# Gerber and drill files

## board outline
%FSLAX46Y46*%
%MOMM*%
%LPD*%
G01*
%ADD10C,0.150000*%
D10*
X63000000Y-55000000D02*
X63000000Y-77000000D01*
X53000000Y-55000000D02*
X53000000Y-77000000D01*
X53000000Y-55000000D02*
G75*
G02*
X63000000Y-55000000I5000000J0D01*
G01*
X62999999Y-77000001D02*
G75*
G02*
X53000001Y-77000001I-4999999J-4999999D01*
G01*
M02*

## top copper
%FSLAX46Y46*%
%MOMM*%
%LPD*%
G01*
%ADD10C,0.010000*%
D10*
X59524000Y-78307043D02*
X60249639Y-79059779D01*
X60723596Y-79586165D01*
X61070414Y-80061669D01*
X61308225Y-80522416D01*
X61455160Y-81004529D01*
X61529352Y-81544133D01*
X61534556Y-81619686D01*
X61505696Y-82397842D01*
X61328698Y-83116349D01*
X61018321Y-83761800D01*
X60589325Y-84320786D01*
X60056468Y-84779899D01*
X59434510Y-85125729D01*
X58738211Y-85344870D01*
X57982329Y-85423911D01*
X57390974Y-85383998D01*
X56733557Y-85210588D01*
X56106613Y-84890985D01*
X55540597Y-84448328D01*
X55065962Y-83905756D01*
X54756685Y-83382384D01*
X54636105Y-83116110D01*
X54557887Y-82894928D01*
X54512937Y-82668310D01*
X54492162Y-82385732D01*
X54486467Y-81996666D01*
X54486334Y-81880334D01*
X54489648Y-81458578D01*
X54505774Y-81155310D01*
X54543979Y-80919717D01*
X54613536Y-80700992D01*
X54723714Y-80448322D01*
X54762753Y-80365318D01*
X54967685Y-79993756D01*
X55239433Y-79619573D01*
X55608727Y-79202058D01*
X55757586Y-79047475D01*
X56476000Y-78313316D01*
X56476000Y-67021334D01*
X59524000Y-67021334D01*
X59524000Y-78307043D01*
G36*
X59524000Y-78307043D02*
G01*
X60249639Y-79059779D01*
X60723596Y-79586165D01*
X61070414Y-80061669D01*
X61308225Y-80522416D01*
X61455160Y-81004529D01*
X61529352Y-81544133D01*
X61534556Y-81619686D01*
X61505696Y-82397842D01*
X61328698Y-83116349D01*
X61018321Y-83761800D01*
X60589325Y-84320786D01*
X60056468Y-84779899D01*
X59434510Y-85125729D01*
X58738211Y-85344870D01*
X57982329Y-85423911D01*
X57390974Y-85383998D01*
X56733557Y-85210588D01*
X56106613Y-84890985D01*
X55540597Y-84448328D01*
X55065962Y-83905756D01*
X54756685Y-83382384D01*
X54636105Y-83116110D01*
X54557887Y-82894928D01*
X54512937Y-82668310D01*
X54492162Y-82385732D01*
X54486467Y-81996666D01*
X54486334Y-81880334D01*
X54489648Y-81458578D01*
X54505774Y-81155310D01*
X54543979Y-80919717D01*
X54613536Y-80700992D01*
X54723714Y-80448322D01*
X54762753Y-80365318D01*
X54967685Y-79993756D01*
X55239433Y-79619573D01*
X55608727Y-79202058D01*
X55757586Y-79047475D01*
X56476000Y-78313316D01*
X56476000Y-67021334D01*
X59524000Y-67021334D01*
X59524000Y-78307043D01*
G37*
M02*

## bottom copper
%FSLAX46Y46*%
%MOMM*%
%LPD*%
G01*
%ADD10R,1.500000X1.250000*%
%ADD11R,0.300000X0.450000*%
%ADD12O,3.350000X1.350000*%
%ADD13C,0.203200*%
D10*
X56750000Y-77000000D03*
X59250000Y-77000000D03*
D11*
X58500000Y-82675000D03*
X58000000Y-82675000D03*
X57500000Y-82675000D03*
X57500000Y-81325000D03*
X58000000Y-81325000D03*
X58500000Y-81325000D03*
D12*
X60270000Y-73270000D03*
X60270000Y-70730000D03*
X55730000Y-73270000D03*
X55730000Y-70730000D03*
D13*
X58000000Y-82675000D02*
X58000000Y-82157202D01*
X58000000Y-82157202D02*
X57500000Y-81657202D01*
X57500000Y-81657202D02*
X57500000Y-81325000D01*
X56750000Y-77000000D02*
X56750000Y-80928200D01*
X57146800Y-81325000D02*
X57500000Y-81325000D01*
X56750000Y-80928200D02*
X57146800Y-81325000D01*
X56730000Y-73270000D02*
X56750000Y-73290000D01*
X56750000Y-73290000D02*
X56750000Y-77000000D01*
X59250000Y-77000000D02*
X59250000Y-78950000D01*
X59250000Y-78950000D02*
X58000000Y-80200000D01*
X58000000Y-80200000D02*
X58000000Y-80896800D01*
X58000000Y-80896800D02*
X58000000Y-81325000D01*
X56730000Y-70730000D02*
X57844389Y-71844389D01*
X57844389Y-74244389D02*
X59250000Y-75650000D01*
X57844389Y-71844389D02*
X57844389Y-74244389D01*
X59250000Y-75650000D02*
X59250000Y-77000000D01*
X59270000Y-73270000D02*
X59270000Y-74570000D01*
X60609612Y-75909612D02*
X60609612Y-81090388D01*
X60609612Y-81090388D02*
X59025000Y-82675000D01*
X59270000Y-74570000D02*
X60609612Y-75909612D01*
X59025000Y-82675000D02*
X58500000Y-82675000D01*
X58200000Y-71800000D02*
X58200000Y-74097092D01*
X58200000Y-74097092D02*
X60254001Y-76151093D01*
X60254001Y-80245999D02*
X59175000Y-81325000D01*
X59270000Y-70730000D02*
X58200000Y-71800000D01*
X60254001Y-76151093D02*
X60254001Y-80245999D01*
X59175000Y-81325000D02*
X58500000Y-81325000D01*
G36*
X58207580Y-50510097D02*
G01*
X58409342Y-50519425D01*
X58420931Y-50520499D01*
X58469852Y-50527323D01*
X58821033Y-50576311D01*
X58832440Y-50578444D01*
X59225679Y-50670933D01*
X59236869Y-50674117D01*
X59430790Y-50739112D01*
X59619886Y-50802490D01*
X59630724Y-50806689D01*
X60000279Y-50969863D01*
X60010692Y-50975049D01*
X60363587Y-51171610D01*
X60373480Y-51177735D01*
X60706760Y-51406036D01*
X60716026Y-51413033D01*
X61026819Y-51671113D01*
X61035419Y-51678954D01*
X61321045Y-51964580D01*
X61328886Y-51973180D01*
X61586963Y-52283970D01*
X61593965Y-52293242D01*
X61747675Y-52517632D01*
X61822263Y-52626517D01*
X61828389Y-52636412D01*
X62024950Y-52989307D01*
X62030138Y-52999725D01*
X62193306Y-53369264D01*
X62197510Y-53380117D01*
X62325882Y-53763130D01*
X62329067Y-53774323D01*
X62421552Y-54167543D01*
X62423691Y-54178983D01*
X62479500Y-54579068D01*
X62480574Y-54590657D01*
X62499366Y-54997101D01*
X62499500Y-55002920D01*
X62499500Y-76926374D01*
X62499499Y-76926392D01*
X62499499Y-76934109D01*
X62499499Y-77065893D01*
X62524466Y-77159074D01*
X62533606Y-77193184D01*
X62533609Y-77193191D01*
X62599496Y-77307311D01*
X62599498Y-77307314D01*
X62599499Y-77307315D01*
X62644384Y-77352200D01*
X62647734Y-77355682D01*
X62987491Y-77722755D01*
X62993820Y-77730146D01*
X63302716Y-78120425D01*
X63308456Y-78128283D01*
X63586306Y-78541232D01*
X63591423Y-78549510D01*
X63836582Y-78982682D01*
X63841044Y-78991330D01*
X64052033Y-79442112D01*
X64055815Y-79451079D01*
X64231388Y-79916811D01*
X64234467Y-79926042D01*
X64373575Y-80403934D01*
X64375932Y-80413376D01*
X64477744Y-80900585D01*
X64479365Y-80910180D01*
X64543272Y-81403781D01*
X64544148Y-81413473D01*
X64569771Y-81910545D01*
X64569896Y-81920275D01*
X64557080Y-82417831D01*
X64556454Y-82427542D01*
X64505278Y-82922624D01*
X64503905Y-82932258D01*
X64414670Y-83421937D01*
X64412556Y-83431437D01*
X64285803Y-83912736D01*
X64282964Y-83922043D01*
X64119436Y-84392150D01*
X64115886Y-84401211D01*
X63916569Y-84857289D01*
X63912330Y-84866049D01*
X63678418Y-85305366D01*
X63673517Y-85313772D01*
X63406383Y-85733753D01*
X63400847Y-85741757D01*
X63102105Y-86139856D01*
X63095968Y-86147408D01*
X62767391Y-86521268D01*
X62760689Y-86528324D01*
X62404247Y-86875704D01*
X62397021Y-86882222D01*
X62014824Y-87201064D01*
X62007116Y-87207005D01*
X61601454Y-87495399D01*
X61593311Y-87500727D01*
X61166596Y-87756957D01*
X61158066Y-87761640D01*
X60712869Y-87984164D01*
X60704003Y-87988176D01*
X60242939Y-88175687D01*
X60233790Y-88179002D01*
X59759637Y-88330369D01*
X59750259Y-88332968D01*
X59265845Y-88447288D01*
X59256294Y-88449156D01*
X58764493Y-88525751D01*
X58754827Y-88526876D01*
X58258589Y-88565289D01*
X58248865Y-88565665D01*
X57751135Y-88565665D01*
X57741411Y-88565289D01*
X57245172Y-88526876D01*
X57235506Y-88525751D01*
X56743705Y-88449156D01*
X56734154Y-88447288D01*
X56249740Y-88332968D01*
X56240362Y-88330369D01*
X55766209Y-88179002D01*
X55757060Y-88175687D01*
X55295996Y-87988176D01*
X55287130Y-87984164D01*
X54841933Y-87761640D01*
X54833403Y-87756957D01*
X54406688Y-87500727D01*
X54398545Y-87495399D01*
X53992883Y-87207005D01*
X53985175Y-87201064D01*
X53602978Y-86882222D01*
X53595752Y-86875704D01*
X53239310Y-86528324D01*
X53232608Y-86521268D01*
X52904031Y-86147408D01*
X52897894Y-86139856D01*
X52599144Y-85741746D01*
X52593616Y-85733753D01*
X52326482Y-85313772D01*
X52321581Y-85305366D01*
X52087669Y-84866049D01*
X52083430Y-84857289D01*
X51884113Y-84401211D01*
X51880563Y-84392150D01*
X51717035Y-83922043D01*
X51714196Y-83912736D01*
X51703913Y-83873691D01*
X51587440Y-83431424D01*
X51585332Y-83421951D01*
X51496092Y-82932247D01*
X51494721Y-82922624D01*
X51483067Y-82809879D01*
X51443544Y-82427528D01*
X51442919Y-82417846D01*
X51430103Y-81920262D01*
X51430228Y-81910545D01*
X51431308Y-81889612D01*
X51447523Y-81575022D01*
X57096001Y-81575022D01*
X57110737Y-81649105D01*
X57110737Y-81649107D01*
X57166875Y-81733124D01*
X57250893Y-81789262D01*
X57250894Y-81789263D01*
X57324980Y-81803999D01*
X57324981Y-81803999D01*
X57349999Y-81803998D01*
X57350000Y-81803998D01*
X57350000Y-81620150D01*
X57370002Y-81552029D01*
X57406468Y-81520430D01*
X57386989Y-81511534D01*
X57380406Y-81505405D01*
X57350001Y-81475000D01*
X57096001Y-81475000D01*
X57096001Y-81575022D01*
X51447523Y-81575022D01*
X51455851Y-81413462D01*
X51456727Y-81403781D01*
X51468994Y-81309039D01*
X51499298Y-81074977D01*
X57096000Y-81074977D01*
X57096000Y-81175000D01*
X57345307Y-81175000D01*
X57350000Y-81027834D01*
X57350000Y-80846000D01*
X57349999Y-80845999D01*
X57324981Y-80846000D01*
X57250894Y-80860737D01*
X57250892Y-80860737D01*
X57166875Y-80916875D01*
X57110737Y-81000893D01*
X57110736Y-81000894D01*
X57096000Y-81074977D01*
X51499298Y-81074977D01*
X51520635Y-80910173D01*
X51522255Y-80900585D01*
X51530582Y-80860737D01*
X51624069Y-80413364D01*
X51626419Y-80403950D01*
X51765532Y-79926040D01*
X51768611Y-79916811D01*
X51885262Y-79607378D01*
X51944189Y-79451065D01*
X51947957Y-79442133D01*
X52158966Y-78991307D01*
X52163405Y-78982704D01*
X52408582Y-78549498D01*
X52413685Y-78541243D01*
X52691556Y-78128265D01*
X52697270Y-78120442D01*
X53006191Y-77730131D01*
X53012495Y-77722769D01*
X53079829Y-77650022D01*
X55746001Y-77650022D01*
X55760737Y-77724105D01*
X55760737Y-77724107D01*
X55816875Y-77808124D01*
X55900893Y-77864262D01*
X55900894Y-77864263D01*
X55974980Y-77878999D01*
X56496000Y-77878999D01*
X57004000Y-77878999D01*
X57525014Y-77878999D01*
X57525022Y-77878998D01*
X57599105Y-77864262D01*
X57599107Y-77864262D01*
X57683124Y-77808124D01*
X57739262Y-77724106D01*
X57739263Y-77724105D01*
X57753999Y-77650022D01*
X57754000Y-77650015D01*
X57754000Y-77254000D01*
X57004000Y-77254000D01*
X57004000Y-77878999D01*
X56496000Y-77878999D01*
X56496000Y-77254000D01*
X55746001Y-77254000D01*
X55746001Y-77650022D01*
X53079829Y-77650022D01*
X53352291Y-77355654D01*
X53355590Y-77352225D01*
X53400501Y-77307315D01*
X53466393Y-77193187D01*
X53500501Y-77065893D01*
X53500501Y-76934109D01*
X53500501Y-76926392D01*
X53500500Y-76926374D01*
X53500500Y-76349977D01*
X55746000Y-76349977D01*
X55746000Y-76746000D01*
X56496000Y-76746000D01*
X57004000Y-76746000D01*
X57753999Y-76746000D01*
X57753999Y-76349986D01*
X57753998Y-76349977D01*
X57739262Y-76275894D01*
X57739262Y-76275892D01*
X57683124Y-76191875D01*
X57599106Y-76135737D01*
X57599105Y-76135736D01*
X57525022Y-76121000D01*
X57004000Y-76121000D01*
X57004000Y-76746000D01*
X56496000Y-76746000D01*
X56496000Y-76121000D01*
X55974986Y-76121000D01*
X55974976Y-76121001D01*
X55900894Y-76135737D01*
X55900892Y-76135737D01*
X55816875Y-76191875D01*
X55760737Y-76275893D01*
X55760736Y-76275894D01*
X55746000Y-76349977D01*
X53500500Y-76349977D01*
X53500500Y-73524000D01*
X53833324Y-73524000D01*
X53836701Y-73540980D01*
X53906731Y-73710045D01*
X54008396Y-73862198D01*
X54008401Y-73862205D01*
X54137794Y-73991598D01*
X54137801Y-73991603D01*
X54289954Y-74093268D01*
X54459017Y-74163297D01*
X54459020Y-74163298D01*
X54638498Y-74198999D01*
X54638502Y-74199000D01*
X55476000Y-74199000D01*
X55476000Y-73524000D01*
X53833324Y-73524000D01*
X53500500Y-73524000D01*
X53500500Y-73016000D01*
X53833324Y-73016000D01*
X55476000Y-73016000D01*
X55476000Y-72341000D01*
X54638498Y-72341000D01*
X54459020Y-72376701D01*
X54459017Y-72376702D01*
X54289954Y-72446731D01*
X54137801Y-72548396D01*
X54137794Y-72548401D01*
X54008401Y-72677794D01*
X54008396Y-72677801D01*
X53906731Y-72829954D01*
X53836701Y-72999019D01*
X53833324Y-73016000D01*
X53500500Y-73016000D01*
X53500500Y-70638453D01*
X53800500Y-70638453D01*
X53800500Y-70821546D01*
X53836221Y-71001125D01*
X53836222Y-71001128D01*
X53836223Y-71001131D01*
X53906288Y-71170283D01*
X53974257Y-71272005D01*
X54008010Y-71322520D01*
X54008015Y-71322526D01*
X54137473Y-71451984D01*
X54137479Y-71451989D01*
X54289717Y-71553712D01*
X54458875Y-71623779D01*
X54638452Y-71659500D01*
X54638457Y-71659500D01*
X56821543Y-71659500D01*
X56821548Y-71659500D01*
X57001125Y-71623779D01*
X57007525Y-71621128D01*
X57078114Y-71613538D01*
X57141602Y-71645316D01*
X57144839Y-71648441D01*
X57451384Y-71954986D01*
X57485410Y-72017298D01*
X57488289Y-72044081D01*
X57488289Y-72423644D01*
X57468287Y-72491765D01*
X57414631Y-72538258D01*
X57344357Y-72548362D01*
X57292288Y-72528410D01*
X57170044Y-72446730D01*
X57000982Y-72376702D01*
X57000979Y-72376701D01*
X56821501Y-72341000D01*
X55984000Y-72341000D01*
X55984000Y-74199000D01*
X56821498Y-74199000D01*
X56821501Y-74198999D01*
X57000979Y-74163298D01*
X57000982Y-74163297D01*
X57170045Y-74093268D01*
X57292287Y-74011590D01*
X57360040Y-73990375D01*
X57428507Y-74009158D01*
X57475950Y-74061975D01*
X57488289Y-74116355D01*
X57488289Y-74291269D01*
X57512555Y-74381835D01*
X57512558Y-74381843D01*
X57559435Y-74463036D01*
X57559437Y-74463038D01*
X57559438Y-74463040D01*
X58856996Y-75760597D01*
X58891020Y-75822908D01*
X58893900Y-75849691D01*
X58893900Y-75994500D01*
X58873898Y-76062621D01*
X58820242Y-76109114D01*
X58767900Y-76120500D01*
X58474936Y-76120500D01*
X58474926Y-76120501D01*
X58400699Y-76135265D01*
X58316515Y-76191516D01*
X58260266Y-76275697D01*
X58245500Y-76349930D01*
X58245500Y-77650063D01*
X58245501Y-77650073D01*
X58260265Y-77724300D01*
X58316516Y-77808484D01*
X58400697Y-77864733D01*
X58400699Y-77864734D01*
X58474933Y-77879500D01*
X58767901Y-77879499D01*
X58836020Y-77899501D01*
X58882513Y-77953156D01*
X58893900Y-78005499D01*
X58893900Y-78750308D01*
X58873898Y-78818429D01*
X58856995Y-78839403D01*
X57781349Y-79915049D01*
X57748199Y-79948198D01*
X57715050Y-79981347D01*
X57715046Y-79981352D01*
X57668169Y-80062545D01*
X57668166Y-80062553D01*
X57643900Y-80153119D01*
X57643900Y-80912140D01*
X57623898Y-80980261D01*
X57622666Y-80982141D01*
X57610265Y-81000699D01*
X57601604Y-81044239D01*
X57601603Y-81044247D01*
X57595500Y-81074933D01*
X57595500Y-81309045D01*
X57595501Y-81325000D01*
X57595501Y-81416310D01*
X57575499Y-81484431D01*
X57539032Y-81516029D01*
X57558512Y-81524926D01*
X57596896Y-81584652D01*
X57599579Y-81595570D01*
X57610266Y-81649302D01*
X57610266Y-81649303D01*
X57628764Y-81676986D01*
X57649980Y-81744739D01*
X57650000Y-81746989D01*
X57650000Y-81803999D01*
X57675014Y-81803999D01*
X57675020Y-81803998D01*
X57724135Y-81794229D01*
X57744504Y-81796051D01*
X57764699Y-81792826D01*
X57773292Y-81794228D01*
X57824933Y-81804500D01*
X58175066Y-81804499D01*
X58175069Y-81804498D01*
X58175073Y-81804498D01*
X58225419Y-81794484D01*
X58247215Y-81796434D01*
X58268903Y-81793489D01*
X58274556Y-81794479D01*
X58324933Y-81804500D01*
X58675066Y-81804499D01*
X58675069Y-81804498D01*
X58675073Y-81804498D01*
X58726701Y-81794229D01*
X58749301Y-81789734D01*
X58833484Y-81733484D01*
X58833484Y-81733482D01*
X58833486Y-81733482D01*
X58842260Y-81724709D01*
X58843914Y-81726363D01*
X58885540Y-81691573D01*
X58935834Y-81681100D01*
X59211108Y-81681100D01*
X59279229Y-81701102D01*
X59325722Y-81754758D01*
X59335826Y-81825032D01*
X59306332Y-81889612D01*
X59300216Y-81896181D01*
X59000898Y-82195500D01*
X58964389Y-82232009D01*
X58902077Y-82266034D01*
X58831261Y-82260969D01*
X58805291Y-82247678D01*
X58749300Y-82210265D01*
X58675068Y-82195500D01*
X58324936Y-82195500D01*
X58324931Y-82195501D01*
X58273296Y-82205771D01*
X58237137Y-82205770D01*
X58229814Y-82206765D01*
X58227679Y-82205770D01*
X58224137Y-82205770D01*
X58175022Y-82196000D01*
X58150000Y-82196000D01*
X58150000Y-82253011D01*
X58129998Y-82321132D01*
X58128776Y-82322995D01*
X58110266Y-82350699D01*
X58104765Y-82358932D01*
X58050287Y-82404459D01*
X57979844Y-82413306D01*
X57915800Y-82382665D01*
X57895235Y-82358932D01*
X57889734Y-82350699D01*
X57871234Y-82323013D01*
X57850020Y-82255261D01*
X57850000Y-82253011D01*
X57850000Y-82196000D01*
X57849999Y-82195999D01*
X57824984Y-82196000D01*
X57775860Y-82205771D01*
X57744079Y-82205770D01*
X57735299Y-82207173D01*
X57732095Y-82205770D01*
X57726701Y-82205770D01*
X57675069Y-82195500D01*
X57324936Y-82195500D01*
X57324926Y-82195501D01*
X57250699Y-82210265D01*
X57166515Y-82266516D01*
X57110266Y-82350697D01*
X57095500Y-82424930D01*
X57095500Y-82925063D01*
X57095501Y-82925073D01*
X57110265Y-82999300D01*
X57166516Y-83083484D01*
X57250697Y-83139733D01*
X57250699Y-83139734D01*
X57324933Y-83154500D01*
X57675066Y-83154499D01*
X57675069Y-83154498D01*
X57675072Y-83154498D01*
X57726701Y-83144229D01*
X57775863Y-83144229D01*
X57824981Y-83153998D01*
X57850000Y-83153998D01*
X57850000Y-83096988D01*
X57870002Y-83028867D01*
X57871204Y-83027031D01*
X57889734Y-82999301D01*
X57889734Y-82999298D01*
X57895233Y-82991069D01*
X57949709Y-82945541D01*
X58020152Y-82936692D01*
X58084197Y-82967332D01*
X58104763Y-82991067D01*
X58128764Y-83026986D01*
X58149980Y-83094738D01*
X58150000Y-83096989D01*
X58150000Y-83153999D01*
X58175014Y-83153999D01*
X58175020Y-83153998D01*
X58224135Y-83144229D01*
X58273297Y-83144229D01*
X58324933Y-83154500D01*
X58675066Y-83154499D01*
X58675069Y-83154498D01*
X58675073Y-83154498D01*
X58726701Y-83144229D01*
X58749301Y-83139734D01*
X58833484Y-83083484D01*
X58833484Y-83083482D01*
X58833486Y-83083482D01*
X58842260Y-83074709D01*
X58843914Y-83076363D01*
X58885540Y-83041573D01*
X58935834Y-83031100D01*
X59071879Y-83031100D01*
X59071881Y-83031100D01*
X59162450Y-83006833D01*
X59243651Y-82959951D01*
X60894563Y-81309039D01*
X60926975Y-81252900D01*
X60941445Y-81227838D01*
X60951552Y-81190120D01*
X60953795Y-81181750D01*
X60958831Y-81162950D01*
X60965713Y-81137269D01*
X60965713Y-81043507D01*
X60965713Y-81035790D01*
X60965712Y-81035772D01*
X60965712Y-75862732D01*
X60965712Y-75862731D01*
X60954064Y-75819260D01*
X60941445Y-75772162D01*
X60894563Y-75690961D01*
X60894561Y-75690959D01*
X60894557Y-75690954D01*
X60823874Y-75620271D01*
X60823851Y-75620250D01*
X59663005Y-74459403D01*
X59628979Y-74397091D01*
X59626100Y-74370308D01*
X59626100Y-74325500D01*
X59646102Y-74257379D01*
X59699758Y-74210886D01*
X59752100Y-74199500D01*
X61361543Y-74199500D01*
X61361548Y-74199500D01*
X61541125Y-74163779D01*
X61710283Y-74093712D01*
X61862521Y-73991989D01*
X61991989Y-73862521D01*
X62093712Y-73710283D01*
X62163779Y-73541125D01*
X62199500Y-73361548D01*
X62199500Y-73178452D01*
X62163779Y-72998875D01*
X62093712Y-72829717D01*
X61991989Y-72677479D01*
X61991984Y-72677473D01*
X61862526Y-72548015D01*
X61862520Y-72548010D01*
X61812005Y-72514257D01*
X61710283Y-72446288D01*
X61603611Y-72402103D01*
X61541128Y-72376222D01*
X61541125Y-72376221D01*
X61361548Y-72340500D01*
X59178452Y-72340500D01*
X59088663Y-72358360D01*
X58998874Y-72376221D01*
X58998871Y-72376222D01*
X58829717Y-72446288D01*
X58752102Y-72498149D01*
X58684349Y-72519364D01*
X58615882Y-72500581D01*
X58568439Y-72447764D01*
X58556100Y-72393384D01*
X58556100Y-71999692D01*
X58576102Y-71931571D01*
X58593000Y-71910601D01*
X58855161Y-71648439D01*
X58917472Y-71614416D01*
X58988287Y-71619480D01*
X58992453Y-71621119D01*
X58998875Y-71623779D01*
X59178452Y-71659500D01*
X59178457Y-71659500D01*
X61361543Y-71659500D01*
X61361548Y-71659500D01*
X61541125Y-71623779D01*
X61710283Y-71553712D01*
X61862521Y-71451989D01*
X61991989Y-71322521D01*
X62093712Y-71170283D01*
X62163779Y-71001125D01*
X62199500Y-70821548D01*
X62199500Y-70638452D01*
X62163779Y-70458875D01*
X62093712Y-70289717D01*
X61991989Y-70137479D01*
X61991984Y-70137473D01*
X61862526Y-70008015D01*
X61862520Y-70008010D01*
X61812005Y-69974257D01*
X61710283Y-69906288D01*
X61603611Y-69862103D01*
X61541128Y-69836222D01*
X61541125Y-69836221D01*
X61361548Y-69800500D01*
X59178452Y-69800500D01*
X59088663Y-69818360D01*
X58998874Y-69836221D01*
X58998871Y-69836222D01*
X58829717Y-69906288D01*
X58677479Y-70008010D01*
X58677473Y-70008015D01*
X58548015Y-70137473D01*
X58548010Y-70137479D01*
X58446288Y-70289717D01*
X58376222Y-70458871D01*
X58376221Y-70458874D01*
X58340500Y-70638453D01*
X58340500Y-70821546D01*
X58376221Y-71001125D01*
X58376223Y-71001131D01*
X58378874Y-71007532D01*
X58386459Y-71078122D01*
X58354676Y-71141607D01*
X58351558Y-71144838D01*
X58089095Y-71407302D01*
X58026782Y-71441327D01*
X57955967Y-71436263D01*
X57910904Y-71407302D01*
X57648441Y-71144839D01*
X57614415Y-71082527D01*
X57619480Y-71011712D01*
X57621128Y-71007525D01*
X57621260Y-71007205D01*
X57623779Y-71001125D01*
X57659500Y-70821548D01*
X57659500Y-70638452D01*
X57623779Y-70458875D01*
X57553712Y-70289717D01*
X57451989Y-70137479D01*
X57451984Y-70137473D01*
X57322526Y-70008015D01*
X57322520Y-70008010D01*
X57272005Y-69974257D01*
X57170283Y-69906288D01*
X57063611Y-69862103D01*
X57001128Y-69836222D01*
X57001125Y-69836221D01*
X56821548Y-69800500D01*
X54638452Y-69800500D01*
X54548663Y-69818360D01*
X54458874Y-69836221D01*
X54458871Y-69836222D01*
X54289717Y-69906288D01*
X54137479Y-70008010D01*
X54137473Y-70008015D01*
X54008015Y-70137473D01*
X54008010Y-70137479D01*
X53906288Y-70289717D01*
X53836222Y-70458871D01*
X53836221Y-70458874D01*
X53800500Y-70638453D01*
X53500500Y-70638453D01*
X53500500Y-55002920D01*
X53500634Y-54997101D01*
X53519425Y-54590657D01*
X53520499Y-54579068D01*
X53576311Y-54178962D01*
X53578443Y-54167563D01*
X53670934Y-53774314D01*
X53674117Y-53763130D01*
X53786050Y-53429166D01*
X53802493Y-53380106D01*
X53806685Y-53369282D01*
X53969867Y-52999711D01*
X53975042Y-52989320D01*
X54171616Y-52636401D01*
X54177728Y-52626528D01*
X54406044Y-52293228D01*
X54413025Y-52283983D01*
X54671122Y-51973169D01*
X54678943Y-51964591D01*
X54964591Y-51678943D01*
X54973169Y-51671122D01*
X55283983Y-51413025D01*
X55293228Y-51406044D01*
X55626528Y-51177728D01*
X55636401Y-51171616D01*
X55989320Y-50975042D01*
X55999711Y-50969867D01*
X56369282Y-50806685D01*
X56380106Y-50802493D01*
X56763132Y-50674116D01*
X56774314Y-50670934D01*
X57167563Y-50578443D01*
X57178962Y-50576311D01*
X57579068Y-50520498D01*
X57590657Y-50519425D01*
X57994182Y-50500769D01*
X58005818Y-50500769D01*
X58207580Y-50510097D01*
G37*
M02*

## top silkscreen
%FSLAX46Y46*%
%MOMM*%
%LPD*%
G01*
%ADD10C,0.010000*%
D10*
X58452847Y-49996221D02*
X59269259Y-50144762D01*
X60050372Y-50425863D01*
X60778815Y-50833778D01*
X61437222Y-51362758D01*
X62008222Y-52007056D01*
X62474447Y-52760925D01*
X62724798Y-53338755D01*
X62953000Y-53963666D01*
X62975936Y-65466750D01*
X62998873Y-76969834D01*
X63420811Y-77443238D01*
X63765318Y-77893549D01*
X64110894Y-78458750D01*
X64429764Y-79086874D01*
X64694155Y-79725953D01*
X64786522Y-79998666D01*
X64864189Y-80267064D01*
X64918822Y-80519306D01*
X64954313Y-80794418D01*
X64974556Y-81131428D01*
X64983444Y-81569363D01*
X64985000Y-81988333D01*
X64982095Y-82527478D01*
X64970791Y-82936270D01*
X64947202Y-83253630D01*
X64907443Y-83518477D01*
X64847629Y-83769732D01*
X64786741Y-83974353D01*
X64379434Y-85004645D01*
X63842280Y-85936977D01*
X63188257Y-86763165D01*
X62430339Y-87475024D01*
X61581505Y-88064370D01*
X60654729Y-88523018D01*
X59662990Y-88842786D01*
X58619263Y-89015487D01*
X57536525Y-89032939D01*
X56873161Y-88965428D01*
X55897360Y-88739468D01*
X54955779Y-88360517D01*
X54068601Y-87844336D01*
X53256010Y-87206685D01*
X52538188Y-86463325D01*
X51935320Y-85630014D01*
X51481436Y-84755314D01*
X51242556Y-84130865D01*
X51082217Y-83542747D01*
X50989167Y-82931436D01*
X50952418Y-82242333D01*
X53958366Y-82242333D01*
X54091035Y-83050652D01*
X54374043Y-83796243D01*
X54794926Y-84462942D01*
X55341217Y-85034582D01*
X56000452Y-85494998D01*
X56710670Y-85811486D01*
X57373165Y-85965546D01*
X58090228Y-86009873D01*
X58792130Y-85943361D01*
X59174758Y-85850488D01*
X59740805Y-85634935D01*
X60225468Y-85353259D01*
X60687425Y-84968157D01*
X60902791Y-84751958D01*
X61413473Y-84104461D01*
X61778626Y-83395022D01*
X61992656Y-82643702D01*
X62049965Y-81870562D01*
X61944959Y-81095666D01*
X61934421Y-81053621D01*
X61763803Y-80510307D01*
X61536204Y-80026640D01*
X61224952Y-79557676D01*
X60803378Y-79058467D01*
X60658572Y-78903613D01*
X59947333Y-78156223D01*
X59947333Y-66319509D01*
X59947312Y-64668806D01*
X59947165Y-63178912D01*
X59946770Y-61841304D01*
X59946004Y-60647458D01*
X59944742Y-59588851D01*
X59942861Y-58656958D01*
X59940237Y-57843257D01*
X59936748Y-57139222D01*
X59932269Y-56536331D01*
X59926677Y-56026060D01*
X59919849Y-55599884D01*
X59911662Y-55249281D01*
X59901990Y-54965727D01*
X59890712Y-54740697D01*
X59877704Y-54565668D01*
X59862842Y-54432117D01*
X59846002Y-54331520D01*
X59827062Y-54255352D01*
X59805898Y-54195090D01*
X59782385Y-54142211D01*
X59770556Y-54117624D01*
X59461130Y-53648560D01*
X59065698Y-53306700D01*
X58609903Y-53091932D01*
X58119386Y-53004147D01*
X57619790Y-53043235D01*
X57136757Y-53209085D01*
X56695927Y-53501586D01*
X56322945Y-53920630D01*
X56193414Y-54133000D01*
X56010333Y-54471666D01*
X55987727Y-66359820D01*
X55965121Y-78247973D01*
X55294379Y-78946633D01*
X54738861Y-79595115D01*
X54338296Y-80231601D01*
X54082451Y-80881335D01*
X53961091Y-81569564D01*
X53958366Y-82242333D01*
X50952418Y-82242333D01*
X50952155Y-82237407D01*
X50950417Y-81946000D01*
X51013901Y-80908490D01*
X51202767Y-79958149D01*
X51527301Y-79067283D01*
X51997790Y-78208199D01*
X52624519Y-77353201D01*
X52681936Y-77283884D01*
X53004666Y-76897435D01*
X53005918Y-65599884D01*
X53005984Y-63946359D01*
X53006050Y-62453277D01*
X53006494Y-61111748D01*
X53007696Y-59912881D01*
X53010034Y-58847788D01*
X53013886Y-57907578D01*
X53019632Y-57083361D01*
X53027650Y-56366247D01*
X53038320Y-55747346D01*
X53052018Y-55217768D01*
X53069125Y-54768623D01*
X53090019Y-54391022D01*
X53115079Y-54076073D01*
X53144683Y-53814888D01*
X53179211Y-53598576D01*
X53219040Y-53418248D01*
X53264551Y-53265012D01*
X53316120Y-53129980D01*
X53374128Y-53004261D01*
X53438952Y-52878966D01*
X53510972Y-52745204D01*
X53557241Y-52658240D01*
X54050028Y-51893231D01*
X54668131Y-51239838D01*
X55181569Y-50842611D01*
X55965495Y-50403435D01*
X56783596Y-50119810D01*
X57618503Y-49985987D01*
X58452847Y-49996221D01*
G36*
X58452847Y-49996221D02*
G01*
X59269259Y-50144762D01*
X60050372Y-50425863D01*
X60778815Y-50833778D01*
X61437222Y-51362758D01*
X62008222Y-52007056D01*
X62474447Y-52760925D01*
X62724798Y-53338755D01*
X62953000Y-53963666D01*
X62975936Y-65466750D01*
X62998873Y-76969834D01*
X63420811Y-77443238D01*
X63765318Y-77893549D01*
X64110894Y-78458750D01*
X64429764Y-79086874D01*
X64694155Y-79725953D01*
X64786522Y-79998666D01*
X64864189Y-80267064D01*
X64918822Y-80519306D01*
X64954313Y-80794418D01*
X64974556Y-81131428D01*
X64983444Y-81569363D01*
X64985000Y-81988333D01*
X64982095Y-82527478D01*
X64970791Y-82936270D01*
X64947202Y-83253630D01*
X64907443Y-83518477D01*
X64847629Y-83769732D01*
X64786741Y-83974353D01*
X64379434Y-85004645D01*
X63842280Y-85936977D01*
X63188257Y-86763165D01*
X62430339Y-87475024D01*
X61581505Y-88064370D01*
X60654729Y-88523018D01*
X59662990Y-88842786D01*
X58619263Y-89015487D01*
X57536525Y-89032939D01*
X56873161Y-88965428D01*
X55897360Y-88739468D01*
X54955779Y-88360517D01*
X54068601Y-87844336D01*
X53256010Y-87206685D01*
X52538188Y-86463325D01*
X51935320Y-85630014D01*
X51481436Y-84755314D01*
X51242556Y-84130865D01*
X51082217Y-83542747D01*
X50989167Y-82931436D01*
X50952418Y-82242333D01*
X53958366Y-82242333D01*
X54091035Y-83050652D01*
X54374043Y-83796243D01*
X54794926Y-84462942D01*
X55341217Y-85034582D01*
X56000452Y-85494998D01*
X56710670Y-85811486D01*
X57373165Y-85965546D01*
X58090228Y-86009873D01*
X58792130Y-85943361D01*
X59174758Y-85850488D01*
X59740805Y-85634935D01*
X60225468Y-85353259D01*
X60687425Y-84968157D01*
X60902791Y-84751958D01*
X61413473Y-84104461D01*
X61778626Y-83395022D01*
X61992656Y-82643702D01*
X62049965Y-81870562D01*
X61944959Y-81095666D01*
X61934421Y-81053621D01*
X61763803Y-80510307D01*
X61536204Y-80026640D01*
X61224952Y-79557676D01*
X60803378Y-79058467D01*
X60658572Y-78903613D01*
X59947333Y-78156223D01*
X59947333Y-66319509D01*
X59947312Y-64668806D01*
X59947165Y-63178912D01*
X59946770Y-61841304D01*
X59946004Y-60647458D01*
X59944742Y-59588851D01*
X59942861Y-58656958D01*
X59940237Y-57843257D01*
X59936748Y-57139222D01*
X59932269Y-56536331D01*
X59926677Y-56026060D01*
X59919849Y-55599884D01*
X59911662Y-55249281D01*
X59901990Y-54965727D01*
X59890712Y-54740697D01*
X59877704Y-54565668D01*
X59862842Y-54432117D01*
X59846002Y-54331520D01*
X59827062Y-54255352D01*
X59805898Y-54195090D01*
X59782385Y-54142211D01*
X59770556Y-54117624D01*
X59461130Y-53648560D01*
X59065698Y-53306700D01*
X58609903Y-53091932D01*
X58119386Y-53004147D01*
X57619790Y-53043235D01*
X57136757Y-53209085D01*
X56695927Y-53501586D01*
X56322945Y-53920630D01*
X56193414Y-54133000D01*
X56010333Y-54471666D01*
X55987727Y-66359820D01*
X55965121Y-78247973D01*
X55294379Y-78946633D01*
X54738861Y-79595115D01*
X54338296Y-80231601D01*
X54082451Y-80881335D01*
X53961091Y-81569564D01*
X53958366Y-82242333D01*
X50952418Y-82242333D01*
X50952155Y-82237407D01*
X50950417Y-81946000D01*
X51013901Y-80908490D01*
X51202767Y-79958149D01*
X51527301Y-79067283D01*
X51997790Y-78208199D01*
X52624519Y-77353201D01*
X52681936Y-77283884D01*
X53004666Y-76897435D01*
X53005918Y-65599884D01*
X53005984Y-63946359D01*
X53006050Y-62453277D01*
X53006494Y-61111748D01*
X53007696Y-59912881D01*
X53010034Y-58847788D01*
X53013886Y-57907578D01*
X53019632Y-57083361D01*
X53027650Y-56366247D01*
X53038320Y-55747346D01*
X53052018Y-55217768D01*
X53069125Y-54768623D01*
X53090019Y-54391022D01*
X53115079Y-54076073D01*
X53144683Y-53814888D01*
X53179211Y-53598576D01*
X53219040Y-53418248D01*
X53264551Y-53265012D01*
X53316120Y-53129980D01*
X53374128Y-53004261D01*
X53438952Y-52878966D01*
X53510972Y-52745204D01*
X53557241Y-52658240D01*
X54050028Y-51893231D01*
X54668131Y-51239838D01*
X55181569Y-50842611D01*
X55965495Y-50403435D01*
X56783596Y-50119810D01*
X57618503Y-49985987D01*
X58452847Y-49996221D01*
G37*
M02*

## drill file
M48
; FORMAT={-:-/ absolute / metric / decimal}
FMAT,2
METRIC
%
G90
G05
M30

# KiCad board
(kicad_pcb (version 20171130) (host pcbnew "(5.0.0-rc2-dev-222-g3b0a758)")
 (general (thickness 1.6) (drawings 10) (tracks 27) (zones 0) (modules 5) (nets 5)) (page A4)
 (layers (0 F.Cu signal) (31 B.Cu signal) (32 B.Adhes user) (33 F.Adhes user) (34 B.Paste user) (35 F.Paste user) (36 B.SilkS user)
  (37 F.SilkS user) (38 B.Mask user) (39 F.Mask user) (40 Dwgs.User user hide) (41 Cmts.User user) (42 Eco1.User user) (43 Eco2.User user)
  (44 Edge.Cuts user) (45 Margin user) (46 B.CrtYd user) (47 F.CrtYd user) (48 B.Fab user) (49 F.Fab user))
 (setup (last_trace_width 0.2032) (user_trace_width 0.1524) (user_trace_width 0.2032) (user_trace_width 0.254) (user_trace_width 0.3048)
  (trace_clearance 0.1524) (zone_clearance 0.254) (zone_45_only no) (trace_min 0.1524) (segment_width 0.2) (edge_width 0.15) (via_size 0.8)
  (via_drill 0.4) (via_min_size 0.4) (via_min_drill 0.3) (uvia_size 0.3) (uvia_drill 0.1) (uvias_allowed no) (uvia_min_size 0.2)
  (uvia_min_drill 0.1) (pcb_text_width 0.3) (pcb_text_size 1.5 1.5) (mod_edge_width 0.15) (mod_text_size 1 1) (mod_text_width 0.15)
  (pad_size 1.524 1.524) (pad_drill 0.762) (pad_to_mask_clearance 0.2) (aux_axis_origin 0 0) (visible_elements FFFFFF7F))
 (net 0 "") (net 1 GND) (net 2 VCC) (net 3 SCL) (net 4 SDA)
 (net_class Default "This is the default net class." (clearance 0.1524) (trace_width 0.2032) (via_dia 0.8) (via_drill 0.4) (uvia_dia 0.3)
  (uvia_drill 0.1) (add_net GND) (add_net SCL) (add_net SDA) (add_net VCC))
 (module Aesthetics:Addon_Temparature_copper (layer F.Cu) (at 58 76.25)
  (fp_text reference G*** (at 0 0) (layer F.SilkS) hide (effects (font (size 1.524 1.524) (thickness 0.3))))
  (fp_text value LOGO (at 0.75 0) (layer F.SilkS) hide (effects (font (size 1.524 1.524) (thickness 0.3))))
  (fp_poly
   (pts (xy 1.524 2.057043) (xy 2.249639 2.809779) (xy 2.723596 3.336165) (xy 3.070414 3.811669) (xy 3.308225 4.272416)
    (xy 3.45516 4.754529) (xy 3.529352 5.294133) (xy 3.534556 5.369686) (xy 3.505696 6.147842) (xy 3.328698 6.866349) (xy 3.018321 7.5118)
    (xy 2.589325 8.070786) (xy 2.056468 8.529899) (xy 1.43451 8.875729) (xy 0.738211 9.09487) (xy -0.017671 9.173911)
    (xy -0.609026 9.133998) (xy -1.266443 8.960588) (xy -1.893387 8.640985) (xy -2.459403 8.198328) (xy -2.934038 7.655756)
    (xy -3.243315 7.132384) (xy -3.363895 6.86611) (xy -3.442113 6.644928) (xy -3.487063 6.41831) (xy -3.507838 6.135732)
    (xy -3.513533 5.746666) (xy -3.513666 5.630334) (xy -3.510352 5.208578) (xy -3.494226 4.90531) (xy -3.456021 4.669717)
    (xy -3.386464 4.450992) (xy -3.276286 4.198322) (xy -3.237247 4.115318) (xy -3.032315 3.743756) (xy -2.760567 3.369573)
    (xy -2.391273 2.952058) (xy -2.242414 2.797475) (xy -1.524 2.063316) (xy -1.524 -9.228666) (xy 1.524 -9.228666) (xy 1.524 2.057043))
   (layer F.Cu) (width 0.01)))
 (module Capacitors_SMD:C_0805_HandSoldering (layer B.Cu) (at 58 77 180)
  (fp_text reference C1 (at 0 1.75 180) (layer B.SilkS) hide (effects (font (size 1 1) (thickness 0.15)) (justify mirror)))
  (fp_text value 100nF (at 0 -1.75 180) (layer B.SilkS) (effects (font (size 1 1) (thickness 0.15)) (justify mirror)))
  (pad 2 smd rect (at 1.25 0 180) (size 1.5 1.25) (layers B.Cu B.Paste B.Mask) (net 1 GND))
  (pad 1 smd rect (at -1.25 0 180) (size 1.5 1.25) (layers B.Cu B.Paste B.Mask) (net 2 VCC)))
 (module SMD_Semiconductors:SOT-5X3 (layer B.Cu) (at 58 82 90)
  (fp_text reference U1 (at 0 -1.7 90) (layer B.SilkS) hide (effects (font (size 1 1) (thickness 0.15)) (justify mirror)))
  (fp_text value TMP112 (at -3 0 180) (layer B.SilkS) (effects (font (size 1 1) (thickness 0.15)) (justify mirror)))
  (pad 1 smd rect (at -0.675 0.5 90) (size 0.45 0.3) (layers B.Cu B.Paste B.Mask) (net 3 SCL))
  (pad 2 smd rect (at -0.675 0 90) (size 0.45 0.3) (layers B.Cu B.Paste B.Mask) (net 1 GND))
  (pad 3 smd rect (at -0.675 -0.5 90) (size 0.45 0.3) (layers B.Cu B.Paste B.Mask))
  (pad 4 smd rect (at 0.675 -0.5 90) (size 0.45 0.3) (layers B.Cu B.Paste B.Mask) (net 1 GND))
  (pad 5 smd rect (at 0.675 0 90) (size 0.45 0.3) (layers B.Cu B.Paste B.Mask) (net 2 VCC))
  (pad 6 smd rect (at 0.675 0.5 90) (size 0.45 0.3) (layers B.Cu B.Paste B.Mask) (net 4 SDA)))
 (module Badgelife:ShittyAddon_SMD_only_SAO (layer F.Cu) (at 56.73 70.73)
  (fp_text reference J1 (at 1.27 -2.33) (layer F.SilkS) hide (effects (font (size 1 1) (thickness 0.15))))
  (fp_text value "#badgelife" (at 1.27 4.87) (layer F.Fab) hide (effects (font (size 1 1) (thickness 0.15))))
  (pad 3 smd oval (at 2.54 2.54) (size 3.35 1.35) (drill (offset 1 0)) (layers B.Cu B.Paste B.Mask) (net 3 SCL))
  (pad 4 smd oval (at 2.54 0) (size 3.35 1.35) (drill (offset 1 0)) (layers B.Cu B.Paste B.Mask) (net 4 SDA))
  (pad 2 smd oval (at 0 2.54) (size 3.35 1.35) (drill (offset -1 0)) (layers B.Cu B.Paste B.Mask) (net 1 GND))
  (pad 1 smd oval (at 0 0) (size 3.35 1.35) (drill (offset -1 0)) (layers B.Cu B.Paste B.Mask) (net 2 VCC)))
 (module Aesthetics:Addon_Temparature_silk (layer F.Cu) (at 58 69.5)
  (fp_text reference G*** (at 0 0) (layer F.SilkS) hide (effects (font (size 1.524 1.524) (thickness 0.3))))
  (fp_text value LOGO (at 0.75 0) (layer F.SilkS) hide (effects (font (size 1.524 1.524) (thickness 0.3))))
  (fp_poly
   (pts (xy 0.452847 -19.503779) (xy 1.269259 -19.355238) (xy 2.050372 -19.074137) (xy 2.778815 -18.666222) (xy 3.437222 -18.137242)
    (xy 4.008222 -17.492944) (xy 4.474447 -16.739075) (xy 4.724798 -16.161245) (xy 4.953 -15.536334) (xy 4.975936 -4.03325)
    (xy 4.998873 7.469834) (xy 5.420811 7.943238) (xy 5.765318 8.393549) (xy 6.110894 8.95875) (xy 6.429764 9.586874)
    (xy 6.694155 10.225953) (xy 6.786522 10.498666) (xy 6.864189 10.767064) (xy 6.918822 11.019306) (xy 6.954313 11.294418)
    (xy 6.974556 11.631428) (xy 6.983444 12.069363) (xy 6.985 12.488333) (xy 6.982095 13.027478) (xy 6.970791 13.43627)
    (xy 6.947202 13.75363) (xy 6.907443 14.018477) (xy 6.847629 14.269732) (xy 6.786741 14.474353) (xy 6.379434 15.504645)
    (xy 5.84228 16.436977) (xy 5.188257 17.263165) (xy 4.430339 17.975024) (xy 3.581505 18.56437) (xy 2.654729 19.023018)
    (xy 1.66299 19.342786) (xy 0.619263 19.515487) (xy -0.463475 19.532939) (xy -1.126839 19.465428) (xy -2.10264 19.239468)
    (xy -3.044221 18.860517) (xy -3.931399 18.344336) (xy -4.74399 17.706685) (xy -5.461812 16.963325) (xy -6.06468 16.130014)
    (xy -6.518564 15.255314) (xy -6.757444 14.630865) (xy -6.917783 14.042747) (xy -7.010833 13.431436) (xy -7.047582 12.742333)
    (xy -4.041634 12.742333) (xy -3.908965 13.550652) (xy -3.625957 14.296243) (xy -3.205074 14.962942) (xy -2.658783 15.534582)
    (xy -1.999548 15.994998) (xy -1.28933 16.311486) (xy -0.626835 16.465546) (xy 0.090228 16.509873) (xy 0.79213 16.443361)
    (xy 1.174758 16.350488) (xy 1.740805 16.134935) (xy 2.225468 15.853259) (xy 2.687425 15.468157) (xy 2.902791 15.251958)
    (xy 3.413473 14.604461) (xy 3.778626 13.895022) (xy 3.992656 13.143702) (xy 4.049965 12.370562) (xy 3.944959 11.595666)
    (xy 3.934421 11.553621) (xy 3.763803 11.010307) (xy 3.536204 10.52664) (xy 3.224952 10.057676) (xy 2.803378 9.558467)
    (xy 2.658572 9.403613) (xy 1.947333 8.656223) (xy 1.947333 -3.180491) (xy 1.947312 -4.831194) (xy 1.947165 -6.321088)
    (xy 1.94677 -7.658696) (xy 1.946004 -8.852542) (xy 1.944742 -9.911149) (xy 1.942861 -10.843042) (xy 1.940237 -11.656743)
    (xy 1.936748 -12.360778) (xy 1.932269 -12.963669) (xy 1.926677 -13.47394) (xy 1.919849 -13.900116) (xy 1.911662 -14.250719)
    (xy 1.90199 -14.534273) (xy 1.890712 -14.759303) (xy 1.877704 -14.934332) (xy 1.862842 -15.067883) (xy 1.846002 -15.16848)
    (xy 1.827062 -15.244648) (xy 1.805898 -15.30491) (xy 1.782385 -15.357789) (xy 1.770556 -15.382376) (xy 1.46113 -15.85144)
    (xy 1.065698 -16.1933) (xy 0.609903 -16.408068) (xy 0.119386 -16.495853) (xy -0.38021 -16.456765) (xy -0.863243 -16.290915)
    (xy -1.304073 -15.998414) (xy -1.677055 -15.57937) (xy -1.806586 -15.367) (xy -1.989667 -15.028334) (xy -2.012273 -3.14018)
    (xy -2.034879 8.747973) (xy -2.705621 9.446633) (xy -3.261139 10.095115) (xy -3.661704 10.731601) (xy -3.917549 11.381335)
    (xy -4.038909 12.069564) (xy -4.041634 12.742333) (xy -7.047582 12.742333) (xy -7.047845 12.737407) (xy -7.049583 12.446)
    (xy -6.986099 11.40849) (xy -6.797233 10.458149) (xy -6.472699 9.567283) (xy -6.00221 8.708199) (xy -5.375481 7.853201)
    (xy -5.318064 7.783884) (xy -4.995334 7.397435) (xy -4.994082 -3.900116) (xy -4.994016 -5.553641) (xy -4.99395 -7.046723)
    (xy -4.993506 -8.388252) (xy -4.992304 -9.587119) (xy -4.989966 -10.652212) (xy -4.986114 -11.592422) (xy -4.980368 -12.416639)
    (xy -4.97235 -13.133753) (xy -4.96168 -13.752654) (xy -4.947982 -14.282232) (xy -4.930875 -14.731377) (xy -4.909981 -15.108978)
    (xy -4.884921 -15.423927) (xy -4.855317 -15.685112) (xy -4.820789 -15.901424) (xy -4.78096 -16.081752) (xy -4.735449 -16.234988)
    (xy -4.68388 -16.37002) (xy -4.625872 -16.495739) (xy -4.561048 -16.621034) (xy -4.489028 -16.754796) (xy -4.442759 -16.84176)
    (xy -3.949972 -17.606769) (xy -3.331869 -18.260162) (xy -2.818431 -18.657389) (xy -2.034505 -19.096565) (xy -1.216404 -19.38019)
    (xy -0.381497 -19.514013) (xy 0.452847 -19.503779))
   (layer F.SilkS) (width 0.01)))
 (gr_line (start 63 55) (end 63 77) (layer Edge.Cuts) (width 0.15))
 (gr_line (start 53 55) (end 53 77) (layer Edge.Cuts) (width 0.15))
 (gr_arc (start 58 55) (end 63 55) (angle -180) (layer Edge.Cuts) (width 0.15))
 (gr_arc (start 58 82) (end 53.000001 77.000001) (angle -270) (layer Edge.Cuts) (width 0.15))
 (segment (start 58 82.675) (end 58 82.157202) (width 0.2032) (layer B.Cu) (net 1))
 (segment (start 58 82.157202) (end 57.5 81.657202) (width 0.2032) (layer B.Cu) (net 1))
 (segment (start 57.5 81.657202) (end 57.5 81.325) (width 0.2032) (layer B.Cu) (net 1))
 (segment (start 56.75 77) (end 56.75 80.9282) (width 0.2032) (layer B.Cu) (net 1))
 (segment (start 57.1468 81.325) (end 57.5 81.325) (width 0.2032) (layer B.Cu) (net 1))
 (segment (start 56.75 80.9282) (end 57.1468 81.325) (width 0.2032) (layer B.Cu) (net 1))
 (segment (start 56.73 73.27) (end 56.75 73.29) (width 0.2032) (layer B.Cu) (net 1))
 (segment (start 56.75 73.29) (end 56.75 77) (width 0.2032) (layer B.Cu) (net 1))
 (segment (start 59.25 77) (end 59.25 78.95) (width 0.2032) (layer B.Cu) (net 2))
 (segment (start 59.25 78.95) (end 58 80.2) (width 0.2032) (layer B.Cu) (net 2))
 (segment (start 58 80.2) (end 58 80.8968) (width 0.2032) (layer B.Cu) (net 2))
 (segment (start 58 80.8968) (end 58 81.325) (width 0.2032) (layer B.Cu) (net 2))
 (segment (start 56.73 70.73) (end 57.844389 71.844389) (width 0.2032) (layer B.Cu) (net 2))
 (segment (start 57.844389 74.244389) (end 59.25 75.65) (width 0.2032) (layer B.Cu) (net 2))
 (segment (start 57.844389 71.844389) (end 57.844389 74.244389) (width 0.2032) (layer B.Cu) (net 2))
 (segment (start 59.25 75.65) (end 59.25 77) (width 0.2032) (layer B.Cu) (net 2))
 (segment (start 59.27 73.27) (end 59.27 74.57) (width 0.2032) (layer B.Cu) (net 3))
 (segment (start 60.609612 75.909612) (end 60.609612 81.090388) (width 0.2032) (layer B.Cu) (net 3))
 (segment (start 60.609612 81.090388) (end 59.025 82.675) (width 0.2032) (layer B.Cu) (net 3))
 (segment (start 59.27 74.57) (end 60.609612 75.909612) (width 0.2032) (layer B.Cu) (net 3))
 (segment (start 59.025 82.675) (end 58.5 82.675) (width 0.2032) (layer B.Cu) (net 3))
 (segment (start 58.2 71.8) (end 58.2 74.097092) (width 0.2032) (layer B.Cu) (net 4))
 (segment (start 58.2 74.097092) (end 60.254001 76.151093) (width 0.2032) (layer B.Cu) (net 4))
 (segment (start 60.254001 80.245999) (end 59.175 81.325) (width 0.2032) (layer B.Cu) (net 4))
 (segment (start 59.27 70.73) (end 58.2 71.8) (width 0.2032) (layer B.Cu) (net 4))
 (segment (start 60.254001 76.151093) (end 60.254001 80.245999) (width 0.2032) (layer B.Cu) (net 4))
 (segment (start 59.175 81.325) (end 58.5 81.325) (width 0.2032) (layer B.Cu) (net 4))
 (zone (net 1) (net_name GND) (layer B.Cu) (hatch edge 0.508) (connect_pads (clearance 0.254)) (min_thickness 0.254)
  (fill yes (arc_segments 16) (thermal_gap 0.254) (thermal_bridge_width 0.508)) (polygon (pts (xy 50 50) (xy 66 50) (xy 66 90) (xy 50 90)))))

